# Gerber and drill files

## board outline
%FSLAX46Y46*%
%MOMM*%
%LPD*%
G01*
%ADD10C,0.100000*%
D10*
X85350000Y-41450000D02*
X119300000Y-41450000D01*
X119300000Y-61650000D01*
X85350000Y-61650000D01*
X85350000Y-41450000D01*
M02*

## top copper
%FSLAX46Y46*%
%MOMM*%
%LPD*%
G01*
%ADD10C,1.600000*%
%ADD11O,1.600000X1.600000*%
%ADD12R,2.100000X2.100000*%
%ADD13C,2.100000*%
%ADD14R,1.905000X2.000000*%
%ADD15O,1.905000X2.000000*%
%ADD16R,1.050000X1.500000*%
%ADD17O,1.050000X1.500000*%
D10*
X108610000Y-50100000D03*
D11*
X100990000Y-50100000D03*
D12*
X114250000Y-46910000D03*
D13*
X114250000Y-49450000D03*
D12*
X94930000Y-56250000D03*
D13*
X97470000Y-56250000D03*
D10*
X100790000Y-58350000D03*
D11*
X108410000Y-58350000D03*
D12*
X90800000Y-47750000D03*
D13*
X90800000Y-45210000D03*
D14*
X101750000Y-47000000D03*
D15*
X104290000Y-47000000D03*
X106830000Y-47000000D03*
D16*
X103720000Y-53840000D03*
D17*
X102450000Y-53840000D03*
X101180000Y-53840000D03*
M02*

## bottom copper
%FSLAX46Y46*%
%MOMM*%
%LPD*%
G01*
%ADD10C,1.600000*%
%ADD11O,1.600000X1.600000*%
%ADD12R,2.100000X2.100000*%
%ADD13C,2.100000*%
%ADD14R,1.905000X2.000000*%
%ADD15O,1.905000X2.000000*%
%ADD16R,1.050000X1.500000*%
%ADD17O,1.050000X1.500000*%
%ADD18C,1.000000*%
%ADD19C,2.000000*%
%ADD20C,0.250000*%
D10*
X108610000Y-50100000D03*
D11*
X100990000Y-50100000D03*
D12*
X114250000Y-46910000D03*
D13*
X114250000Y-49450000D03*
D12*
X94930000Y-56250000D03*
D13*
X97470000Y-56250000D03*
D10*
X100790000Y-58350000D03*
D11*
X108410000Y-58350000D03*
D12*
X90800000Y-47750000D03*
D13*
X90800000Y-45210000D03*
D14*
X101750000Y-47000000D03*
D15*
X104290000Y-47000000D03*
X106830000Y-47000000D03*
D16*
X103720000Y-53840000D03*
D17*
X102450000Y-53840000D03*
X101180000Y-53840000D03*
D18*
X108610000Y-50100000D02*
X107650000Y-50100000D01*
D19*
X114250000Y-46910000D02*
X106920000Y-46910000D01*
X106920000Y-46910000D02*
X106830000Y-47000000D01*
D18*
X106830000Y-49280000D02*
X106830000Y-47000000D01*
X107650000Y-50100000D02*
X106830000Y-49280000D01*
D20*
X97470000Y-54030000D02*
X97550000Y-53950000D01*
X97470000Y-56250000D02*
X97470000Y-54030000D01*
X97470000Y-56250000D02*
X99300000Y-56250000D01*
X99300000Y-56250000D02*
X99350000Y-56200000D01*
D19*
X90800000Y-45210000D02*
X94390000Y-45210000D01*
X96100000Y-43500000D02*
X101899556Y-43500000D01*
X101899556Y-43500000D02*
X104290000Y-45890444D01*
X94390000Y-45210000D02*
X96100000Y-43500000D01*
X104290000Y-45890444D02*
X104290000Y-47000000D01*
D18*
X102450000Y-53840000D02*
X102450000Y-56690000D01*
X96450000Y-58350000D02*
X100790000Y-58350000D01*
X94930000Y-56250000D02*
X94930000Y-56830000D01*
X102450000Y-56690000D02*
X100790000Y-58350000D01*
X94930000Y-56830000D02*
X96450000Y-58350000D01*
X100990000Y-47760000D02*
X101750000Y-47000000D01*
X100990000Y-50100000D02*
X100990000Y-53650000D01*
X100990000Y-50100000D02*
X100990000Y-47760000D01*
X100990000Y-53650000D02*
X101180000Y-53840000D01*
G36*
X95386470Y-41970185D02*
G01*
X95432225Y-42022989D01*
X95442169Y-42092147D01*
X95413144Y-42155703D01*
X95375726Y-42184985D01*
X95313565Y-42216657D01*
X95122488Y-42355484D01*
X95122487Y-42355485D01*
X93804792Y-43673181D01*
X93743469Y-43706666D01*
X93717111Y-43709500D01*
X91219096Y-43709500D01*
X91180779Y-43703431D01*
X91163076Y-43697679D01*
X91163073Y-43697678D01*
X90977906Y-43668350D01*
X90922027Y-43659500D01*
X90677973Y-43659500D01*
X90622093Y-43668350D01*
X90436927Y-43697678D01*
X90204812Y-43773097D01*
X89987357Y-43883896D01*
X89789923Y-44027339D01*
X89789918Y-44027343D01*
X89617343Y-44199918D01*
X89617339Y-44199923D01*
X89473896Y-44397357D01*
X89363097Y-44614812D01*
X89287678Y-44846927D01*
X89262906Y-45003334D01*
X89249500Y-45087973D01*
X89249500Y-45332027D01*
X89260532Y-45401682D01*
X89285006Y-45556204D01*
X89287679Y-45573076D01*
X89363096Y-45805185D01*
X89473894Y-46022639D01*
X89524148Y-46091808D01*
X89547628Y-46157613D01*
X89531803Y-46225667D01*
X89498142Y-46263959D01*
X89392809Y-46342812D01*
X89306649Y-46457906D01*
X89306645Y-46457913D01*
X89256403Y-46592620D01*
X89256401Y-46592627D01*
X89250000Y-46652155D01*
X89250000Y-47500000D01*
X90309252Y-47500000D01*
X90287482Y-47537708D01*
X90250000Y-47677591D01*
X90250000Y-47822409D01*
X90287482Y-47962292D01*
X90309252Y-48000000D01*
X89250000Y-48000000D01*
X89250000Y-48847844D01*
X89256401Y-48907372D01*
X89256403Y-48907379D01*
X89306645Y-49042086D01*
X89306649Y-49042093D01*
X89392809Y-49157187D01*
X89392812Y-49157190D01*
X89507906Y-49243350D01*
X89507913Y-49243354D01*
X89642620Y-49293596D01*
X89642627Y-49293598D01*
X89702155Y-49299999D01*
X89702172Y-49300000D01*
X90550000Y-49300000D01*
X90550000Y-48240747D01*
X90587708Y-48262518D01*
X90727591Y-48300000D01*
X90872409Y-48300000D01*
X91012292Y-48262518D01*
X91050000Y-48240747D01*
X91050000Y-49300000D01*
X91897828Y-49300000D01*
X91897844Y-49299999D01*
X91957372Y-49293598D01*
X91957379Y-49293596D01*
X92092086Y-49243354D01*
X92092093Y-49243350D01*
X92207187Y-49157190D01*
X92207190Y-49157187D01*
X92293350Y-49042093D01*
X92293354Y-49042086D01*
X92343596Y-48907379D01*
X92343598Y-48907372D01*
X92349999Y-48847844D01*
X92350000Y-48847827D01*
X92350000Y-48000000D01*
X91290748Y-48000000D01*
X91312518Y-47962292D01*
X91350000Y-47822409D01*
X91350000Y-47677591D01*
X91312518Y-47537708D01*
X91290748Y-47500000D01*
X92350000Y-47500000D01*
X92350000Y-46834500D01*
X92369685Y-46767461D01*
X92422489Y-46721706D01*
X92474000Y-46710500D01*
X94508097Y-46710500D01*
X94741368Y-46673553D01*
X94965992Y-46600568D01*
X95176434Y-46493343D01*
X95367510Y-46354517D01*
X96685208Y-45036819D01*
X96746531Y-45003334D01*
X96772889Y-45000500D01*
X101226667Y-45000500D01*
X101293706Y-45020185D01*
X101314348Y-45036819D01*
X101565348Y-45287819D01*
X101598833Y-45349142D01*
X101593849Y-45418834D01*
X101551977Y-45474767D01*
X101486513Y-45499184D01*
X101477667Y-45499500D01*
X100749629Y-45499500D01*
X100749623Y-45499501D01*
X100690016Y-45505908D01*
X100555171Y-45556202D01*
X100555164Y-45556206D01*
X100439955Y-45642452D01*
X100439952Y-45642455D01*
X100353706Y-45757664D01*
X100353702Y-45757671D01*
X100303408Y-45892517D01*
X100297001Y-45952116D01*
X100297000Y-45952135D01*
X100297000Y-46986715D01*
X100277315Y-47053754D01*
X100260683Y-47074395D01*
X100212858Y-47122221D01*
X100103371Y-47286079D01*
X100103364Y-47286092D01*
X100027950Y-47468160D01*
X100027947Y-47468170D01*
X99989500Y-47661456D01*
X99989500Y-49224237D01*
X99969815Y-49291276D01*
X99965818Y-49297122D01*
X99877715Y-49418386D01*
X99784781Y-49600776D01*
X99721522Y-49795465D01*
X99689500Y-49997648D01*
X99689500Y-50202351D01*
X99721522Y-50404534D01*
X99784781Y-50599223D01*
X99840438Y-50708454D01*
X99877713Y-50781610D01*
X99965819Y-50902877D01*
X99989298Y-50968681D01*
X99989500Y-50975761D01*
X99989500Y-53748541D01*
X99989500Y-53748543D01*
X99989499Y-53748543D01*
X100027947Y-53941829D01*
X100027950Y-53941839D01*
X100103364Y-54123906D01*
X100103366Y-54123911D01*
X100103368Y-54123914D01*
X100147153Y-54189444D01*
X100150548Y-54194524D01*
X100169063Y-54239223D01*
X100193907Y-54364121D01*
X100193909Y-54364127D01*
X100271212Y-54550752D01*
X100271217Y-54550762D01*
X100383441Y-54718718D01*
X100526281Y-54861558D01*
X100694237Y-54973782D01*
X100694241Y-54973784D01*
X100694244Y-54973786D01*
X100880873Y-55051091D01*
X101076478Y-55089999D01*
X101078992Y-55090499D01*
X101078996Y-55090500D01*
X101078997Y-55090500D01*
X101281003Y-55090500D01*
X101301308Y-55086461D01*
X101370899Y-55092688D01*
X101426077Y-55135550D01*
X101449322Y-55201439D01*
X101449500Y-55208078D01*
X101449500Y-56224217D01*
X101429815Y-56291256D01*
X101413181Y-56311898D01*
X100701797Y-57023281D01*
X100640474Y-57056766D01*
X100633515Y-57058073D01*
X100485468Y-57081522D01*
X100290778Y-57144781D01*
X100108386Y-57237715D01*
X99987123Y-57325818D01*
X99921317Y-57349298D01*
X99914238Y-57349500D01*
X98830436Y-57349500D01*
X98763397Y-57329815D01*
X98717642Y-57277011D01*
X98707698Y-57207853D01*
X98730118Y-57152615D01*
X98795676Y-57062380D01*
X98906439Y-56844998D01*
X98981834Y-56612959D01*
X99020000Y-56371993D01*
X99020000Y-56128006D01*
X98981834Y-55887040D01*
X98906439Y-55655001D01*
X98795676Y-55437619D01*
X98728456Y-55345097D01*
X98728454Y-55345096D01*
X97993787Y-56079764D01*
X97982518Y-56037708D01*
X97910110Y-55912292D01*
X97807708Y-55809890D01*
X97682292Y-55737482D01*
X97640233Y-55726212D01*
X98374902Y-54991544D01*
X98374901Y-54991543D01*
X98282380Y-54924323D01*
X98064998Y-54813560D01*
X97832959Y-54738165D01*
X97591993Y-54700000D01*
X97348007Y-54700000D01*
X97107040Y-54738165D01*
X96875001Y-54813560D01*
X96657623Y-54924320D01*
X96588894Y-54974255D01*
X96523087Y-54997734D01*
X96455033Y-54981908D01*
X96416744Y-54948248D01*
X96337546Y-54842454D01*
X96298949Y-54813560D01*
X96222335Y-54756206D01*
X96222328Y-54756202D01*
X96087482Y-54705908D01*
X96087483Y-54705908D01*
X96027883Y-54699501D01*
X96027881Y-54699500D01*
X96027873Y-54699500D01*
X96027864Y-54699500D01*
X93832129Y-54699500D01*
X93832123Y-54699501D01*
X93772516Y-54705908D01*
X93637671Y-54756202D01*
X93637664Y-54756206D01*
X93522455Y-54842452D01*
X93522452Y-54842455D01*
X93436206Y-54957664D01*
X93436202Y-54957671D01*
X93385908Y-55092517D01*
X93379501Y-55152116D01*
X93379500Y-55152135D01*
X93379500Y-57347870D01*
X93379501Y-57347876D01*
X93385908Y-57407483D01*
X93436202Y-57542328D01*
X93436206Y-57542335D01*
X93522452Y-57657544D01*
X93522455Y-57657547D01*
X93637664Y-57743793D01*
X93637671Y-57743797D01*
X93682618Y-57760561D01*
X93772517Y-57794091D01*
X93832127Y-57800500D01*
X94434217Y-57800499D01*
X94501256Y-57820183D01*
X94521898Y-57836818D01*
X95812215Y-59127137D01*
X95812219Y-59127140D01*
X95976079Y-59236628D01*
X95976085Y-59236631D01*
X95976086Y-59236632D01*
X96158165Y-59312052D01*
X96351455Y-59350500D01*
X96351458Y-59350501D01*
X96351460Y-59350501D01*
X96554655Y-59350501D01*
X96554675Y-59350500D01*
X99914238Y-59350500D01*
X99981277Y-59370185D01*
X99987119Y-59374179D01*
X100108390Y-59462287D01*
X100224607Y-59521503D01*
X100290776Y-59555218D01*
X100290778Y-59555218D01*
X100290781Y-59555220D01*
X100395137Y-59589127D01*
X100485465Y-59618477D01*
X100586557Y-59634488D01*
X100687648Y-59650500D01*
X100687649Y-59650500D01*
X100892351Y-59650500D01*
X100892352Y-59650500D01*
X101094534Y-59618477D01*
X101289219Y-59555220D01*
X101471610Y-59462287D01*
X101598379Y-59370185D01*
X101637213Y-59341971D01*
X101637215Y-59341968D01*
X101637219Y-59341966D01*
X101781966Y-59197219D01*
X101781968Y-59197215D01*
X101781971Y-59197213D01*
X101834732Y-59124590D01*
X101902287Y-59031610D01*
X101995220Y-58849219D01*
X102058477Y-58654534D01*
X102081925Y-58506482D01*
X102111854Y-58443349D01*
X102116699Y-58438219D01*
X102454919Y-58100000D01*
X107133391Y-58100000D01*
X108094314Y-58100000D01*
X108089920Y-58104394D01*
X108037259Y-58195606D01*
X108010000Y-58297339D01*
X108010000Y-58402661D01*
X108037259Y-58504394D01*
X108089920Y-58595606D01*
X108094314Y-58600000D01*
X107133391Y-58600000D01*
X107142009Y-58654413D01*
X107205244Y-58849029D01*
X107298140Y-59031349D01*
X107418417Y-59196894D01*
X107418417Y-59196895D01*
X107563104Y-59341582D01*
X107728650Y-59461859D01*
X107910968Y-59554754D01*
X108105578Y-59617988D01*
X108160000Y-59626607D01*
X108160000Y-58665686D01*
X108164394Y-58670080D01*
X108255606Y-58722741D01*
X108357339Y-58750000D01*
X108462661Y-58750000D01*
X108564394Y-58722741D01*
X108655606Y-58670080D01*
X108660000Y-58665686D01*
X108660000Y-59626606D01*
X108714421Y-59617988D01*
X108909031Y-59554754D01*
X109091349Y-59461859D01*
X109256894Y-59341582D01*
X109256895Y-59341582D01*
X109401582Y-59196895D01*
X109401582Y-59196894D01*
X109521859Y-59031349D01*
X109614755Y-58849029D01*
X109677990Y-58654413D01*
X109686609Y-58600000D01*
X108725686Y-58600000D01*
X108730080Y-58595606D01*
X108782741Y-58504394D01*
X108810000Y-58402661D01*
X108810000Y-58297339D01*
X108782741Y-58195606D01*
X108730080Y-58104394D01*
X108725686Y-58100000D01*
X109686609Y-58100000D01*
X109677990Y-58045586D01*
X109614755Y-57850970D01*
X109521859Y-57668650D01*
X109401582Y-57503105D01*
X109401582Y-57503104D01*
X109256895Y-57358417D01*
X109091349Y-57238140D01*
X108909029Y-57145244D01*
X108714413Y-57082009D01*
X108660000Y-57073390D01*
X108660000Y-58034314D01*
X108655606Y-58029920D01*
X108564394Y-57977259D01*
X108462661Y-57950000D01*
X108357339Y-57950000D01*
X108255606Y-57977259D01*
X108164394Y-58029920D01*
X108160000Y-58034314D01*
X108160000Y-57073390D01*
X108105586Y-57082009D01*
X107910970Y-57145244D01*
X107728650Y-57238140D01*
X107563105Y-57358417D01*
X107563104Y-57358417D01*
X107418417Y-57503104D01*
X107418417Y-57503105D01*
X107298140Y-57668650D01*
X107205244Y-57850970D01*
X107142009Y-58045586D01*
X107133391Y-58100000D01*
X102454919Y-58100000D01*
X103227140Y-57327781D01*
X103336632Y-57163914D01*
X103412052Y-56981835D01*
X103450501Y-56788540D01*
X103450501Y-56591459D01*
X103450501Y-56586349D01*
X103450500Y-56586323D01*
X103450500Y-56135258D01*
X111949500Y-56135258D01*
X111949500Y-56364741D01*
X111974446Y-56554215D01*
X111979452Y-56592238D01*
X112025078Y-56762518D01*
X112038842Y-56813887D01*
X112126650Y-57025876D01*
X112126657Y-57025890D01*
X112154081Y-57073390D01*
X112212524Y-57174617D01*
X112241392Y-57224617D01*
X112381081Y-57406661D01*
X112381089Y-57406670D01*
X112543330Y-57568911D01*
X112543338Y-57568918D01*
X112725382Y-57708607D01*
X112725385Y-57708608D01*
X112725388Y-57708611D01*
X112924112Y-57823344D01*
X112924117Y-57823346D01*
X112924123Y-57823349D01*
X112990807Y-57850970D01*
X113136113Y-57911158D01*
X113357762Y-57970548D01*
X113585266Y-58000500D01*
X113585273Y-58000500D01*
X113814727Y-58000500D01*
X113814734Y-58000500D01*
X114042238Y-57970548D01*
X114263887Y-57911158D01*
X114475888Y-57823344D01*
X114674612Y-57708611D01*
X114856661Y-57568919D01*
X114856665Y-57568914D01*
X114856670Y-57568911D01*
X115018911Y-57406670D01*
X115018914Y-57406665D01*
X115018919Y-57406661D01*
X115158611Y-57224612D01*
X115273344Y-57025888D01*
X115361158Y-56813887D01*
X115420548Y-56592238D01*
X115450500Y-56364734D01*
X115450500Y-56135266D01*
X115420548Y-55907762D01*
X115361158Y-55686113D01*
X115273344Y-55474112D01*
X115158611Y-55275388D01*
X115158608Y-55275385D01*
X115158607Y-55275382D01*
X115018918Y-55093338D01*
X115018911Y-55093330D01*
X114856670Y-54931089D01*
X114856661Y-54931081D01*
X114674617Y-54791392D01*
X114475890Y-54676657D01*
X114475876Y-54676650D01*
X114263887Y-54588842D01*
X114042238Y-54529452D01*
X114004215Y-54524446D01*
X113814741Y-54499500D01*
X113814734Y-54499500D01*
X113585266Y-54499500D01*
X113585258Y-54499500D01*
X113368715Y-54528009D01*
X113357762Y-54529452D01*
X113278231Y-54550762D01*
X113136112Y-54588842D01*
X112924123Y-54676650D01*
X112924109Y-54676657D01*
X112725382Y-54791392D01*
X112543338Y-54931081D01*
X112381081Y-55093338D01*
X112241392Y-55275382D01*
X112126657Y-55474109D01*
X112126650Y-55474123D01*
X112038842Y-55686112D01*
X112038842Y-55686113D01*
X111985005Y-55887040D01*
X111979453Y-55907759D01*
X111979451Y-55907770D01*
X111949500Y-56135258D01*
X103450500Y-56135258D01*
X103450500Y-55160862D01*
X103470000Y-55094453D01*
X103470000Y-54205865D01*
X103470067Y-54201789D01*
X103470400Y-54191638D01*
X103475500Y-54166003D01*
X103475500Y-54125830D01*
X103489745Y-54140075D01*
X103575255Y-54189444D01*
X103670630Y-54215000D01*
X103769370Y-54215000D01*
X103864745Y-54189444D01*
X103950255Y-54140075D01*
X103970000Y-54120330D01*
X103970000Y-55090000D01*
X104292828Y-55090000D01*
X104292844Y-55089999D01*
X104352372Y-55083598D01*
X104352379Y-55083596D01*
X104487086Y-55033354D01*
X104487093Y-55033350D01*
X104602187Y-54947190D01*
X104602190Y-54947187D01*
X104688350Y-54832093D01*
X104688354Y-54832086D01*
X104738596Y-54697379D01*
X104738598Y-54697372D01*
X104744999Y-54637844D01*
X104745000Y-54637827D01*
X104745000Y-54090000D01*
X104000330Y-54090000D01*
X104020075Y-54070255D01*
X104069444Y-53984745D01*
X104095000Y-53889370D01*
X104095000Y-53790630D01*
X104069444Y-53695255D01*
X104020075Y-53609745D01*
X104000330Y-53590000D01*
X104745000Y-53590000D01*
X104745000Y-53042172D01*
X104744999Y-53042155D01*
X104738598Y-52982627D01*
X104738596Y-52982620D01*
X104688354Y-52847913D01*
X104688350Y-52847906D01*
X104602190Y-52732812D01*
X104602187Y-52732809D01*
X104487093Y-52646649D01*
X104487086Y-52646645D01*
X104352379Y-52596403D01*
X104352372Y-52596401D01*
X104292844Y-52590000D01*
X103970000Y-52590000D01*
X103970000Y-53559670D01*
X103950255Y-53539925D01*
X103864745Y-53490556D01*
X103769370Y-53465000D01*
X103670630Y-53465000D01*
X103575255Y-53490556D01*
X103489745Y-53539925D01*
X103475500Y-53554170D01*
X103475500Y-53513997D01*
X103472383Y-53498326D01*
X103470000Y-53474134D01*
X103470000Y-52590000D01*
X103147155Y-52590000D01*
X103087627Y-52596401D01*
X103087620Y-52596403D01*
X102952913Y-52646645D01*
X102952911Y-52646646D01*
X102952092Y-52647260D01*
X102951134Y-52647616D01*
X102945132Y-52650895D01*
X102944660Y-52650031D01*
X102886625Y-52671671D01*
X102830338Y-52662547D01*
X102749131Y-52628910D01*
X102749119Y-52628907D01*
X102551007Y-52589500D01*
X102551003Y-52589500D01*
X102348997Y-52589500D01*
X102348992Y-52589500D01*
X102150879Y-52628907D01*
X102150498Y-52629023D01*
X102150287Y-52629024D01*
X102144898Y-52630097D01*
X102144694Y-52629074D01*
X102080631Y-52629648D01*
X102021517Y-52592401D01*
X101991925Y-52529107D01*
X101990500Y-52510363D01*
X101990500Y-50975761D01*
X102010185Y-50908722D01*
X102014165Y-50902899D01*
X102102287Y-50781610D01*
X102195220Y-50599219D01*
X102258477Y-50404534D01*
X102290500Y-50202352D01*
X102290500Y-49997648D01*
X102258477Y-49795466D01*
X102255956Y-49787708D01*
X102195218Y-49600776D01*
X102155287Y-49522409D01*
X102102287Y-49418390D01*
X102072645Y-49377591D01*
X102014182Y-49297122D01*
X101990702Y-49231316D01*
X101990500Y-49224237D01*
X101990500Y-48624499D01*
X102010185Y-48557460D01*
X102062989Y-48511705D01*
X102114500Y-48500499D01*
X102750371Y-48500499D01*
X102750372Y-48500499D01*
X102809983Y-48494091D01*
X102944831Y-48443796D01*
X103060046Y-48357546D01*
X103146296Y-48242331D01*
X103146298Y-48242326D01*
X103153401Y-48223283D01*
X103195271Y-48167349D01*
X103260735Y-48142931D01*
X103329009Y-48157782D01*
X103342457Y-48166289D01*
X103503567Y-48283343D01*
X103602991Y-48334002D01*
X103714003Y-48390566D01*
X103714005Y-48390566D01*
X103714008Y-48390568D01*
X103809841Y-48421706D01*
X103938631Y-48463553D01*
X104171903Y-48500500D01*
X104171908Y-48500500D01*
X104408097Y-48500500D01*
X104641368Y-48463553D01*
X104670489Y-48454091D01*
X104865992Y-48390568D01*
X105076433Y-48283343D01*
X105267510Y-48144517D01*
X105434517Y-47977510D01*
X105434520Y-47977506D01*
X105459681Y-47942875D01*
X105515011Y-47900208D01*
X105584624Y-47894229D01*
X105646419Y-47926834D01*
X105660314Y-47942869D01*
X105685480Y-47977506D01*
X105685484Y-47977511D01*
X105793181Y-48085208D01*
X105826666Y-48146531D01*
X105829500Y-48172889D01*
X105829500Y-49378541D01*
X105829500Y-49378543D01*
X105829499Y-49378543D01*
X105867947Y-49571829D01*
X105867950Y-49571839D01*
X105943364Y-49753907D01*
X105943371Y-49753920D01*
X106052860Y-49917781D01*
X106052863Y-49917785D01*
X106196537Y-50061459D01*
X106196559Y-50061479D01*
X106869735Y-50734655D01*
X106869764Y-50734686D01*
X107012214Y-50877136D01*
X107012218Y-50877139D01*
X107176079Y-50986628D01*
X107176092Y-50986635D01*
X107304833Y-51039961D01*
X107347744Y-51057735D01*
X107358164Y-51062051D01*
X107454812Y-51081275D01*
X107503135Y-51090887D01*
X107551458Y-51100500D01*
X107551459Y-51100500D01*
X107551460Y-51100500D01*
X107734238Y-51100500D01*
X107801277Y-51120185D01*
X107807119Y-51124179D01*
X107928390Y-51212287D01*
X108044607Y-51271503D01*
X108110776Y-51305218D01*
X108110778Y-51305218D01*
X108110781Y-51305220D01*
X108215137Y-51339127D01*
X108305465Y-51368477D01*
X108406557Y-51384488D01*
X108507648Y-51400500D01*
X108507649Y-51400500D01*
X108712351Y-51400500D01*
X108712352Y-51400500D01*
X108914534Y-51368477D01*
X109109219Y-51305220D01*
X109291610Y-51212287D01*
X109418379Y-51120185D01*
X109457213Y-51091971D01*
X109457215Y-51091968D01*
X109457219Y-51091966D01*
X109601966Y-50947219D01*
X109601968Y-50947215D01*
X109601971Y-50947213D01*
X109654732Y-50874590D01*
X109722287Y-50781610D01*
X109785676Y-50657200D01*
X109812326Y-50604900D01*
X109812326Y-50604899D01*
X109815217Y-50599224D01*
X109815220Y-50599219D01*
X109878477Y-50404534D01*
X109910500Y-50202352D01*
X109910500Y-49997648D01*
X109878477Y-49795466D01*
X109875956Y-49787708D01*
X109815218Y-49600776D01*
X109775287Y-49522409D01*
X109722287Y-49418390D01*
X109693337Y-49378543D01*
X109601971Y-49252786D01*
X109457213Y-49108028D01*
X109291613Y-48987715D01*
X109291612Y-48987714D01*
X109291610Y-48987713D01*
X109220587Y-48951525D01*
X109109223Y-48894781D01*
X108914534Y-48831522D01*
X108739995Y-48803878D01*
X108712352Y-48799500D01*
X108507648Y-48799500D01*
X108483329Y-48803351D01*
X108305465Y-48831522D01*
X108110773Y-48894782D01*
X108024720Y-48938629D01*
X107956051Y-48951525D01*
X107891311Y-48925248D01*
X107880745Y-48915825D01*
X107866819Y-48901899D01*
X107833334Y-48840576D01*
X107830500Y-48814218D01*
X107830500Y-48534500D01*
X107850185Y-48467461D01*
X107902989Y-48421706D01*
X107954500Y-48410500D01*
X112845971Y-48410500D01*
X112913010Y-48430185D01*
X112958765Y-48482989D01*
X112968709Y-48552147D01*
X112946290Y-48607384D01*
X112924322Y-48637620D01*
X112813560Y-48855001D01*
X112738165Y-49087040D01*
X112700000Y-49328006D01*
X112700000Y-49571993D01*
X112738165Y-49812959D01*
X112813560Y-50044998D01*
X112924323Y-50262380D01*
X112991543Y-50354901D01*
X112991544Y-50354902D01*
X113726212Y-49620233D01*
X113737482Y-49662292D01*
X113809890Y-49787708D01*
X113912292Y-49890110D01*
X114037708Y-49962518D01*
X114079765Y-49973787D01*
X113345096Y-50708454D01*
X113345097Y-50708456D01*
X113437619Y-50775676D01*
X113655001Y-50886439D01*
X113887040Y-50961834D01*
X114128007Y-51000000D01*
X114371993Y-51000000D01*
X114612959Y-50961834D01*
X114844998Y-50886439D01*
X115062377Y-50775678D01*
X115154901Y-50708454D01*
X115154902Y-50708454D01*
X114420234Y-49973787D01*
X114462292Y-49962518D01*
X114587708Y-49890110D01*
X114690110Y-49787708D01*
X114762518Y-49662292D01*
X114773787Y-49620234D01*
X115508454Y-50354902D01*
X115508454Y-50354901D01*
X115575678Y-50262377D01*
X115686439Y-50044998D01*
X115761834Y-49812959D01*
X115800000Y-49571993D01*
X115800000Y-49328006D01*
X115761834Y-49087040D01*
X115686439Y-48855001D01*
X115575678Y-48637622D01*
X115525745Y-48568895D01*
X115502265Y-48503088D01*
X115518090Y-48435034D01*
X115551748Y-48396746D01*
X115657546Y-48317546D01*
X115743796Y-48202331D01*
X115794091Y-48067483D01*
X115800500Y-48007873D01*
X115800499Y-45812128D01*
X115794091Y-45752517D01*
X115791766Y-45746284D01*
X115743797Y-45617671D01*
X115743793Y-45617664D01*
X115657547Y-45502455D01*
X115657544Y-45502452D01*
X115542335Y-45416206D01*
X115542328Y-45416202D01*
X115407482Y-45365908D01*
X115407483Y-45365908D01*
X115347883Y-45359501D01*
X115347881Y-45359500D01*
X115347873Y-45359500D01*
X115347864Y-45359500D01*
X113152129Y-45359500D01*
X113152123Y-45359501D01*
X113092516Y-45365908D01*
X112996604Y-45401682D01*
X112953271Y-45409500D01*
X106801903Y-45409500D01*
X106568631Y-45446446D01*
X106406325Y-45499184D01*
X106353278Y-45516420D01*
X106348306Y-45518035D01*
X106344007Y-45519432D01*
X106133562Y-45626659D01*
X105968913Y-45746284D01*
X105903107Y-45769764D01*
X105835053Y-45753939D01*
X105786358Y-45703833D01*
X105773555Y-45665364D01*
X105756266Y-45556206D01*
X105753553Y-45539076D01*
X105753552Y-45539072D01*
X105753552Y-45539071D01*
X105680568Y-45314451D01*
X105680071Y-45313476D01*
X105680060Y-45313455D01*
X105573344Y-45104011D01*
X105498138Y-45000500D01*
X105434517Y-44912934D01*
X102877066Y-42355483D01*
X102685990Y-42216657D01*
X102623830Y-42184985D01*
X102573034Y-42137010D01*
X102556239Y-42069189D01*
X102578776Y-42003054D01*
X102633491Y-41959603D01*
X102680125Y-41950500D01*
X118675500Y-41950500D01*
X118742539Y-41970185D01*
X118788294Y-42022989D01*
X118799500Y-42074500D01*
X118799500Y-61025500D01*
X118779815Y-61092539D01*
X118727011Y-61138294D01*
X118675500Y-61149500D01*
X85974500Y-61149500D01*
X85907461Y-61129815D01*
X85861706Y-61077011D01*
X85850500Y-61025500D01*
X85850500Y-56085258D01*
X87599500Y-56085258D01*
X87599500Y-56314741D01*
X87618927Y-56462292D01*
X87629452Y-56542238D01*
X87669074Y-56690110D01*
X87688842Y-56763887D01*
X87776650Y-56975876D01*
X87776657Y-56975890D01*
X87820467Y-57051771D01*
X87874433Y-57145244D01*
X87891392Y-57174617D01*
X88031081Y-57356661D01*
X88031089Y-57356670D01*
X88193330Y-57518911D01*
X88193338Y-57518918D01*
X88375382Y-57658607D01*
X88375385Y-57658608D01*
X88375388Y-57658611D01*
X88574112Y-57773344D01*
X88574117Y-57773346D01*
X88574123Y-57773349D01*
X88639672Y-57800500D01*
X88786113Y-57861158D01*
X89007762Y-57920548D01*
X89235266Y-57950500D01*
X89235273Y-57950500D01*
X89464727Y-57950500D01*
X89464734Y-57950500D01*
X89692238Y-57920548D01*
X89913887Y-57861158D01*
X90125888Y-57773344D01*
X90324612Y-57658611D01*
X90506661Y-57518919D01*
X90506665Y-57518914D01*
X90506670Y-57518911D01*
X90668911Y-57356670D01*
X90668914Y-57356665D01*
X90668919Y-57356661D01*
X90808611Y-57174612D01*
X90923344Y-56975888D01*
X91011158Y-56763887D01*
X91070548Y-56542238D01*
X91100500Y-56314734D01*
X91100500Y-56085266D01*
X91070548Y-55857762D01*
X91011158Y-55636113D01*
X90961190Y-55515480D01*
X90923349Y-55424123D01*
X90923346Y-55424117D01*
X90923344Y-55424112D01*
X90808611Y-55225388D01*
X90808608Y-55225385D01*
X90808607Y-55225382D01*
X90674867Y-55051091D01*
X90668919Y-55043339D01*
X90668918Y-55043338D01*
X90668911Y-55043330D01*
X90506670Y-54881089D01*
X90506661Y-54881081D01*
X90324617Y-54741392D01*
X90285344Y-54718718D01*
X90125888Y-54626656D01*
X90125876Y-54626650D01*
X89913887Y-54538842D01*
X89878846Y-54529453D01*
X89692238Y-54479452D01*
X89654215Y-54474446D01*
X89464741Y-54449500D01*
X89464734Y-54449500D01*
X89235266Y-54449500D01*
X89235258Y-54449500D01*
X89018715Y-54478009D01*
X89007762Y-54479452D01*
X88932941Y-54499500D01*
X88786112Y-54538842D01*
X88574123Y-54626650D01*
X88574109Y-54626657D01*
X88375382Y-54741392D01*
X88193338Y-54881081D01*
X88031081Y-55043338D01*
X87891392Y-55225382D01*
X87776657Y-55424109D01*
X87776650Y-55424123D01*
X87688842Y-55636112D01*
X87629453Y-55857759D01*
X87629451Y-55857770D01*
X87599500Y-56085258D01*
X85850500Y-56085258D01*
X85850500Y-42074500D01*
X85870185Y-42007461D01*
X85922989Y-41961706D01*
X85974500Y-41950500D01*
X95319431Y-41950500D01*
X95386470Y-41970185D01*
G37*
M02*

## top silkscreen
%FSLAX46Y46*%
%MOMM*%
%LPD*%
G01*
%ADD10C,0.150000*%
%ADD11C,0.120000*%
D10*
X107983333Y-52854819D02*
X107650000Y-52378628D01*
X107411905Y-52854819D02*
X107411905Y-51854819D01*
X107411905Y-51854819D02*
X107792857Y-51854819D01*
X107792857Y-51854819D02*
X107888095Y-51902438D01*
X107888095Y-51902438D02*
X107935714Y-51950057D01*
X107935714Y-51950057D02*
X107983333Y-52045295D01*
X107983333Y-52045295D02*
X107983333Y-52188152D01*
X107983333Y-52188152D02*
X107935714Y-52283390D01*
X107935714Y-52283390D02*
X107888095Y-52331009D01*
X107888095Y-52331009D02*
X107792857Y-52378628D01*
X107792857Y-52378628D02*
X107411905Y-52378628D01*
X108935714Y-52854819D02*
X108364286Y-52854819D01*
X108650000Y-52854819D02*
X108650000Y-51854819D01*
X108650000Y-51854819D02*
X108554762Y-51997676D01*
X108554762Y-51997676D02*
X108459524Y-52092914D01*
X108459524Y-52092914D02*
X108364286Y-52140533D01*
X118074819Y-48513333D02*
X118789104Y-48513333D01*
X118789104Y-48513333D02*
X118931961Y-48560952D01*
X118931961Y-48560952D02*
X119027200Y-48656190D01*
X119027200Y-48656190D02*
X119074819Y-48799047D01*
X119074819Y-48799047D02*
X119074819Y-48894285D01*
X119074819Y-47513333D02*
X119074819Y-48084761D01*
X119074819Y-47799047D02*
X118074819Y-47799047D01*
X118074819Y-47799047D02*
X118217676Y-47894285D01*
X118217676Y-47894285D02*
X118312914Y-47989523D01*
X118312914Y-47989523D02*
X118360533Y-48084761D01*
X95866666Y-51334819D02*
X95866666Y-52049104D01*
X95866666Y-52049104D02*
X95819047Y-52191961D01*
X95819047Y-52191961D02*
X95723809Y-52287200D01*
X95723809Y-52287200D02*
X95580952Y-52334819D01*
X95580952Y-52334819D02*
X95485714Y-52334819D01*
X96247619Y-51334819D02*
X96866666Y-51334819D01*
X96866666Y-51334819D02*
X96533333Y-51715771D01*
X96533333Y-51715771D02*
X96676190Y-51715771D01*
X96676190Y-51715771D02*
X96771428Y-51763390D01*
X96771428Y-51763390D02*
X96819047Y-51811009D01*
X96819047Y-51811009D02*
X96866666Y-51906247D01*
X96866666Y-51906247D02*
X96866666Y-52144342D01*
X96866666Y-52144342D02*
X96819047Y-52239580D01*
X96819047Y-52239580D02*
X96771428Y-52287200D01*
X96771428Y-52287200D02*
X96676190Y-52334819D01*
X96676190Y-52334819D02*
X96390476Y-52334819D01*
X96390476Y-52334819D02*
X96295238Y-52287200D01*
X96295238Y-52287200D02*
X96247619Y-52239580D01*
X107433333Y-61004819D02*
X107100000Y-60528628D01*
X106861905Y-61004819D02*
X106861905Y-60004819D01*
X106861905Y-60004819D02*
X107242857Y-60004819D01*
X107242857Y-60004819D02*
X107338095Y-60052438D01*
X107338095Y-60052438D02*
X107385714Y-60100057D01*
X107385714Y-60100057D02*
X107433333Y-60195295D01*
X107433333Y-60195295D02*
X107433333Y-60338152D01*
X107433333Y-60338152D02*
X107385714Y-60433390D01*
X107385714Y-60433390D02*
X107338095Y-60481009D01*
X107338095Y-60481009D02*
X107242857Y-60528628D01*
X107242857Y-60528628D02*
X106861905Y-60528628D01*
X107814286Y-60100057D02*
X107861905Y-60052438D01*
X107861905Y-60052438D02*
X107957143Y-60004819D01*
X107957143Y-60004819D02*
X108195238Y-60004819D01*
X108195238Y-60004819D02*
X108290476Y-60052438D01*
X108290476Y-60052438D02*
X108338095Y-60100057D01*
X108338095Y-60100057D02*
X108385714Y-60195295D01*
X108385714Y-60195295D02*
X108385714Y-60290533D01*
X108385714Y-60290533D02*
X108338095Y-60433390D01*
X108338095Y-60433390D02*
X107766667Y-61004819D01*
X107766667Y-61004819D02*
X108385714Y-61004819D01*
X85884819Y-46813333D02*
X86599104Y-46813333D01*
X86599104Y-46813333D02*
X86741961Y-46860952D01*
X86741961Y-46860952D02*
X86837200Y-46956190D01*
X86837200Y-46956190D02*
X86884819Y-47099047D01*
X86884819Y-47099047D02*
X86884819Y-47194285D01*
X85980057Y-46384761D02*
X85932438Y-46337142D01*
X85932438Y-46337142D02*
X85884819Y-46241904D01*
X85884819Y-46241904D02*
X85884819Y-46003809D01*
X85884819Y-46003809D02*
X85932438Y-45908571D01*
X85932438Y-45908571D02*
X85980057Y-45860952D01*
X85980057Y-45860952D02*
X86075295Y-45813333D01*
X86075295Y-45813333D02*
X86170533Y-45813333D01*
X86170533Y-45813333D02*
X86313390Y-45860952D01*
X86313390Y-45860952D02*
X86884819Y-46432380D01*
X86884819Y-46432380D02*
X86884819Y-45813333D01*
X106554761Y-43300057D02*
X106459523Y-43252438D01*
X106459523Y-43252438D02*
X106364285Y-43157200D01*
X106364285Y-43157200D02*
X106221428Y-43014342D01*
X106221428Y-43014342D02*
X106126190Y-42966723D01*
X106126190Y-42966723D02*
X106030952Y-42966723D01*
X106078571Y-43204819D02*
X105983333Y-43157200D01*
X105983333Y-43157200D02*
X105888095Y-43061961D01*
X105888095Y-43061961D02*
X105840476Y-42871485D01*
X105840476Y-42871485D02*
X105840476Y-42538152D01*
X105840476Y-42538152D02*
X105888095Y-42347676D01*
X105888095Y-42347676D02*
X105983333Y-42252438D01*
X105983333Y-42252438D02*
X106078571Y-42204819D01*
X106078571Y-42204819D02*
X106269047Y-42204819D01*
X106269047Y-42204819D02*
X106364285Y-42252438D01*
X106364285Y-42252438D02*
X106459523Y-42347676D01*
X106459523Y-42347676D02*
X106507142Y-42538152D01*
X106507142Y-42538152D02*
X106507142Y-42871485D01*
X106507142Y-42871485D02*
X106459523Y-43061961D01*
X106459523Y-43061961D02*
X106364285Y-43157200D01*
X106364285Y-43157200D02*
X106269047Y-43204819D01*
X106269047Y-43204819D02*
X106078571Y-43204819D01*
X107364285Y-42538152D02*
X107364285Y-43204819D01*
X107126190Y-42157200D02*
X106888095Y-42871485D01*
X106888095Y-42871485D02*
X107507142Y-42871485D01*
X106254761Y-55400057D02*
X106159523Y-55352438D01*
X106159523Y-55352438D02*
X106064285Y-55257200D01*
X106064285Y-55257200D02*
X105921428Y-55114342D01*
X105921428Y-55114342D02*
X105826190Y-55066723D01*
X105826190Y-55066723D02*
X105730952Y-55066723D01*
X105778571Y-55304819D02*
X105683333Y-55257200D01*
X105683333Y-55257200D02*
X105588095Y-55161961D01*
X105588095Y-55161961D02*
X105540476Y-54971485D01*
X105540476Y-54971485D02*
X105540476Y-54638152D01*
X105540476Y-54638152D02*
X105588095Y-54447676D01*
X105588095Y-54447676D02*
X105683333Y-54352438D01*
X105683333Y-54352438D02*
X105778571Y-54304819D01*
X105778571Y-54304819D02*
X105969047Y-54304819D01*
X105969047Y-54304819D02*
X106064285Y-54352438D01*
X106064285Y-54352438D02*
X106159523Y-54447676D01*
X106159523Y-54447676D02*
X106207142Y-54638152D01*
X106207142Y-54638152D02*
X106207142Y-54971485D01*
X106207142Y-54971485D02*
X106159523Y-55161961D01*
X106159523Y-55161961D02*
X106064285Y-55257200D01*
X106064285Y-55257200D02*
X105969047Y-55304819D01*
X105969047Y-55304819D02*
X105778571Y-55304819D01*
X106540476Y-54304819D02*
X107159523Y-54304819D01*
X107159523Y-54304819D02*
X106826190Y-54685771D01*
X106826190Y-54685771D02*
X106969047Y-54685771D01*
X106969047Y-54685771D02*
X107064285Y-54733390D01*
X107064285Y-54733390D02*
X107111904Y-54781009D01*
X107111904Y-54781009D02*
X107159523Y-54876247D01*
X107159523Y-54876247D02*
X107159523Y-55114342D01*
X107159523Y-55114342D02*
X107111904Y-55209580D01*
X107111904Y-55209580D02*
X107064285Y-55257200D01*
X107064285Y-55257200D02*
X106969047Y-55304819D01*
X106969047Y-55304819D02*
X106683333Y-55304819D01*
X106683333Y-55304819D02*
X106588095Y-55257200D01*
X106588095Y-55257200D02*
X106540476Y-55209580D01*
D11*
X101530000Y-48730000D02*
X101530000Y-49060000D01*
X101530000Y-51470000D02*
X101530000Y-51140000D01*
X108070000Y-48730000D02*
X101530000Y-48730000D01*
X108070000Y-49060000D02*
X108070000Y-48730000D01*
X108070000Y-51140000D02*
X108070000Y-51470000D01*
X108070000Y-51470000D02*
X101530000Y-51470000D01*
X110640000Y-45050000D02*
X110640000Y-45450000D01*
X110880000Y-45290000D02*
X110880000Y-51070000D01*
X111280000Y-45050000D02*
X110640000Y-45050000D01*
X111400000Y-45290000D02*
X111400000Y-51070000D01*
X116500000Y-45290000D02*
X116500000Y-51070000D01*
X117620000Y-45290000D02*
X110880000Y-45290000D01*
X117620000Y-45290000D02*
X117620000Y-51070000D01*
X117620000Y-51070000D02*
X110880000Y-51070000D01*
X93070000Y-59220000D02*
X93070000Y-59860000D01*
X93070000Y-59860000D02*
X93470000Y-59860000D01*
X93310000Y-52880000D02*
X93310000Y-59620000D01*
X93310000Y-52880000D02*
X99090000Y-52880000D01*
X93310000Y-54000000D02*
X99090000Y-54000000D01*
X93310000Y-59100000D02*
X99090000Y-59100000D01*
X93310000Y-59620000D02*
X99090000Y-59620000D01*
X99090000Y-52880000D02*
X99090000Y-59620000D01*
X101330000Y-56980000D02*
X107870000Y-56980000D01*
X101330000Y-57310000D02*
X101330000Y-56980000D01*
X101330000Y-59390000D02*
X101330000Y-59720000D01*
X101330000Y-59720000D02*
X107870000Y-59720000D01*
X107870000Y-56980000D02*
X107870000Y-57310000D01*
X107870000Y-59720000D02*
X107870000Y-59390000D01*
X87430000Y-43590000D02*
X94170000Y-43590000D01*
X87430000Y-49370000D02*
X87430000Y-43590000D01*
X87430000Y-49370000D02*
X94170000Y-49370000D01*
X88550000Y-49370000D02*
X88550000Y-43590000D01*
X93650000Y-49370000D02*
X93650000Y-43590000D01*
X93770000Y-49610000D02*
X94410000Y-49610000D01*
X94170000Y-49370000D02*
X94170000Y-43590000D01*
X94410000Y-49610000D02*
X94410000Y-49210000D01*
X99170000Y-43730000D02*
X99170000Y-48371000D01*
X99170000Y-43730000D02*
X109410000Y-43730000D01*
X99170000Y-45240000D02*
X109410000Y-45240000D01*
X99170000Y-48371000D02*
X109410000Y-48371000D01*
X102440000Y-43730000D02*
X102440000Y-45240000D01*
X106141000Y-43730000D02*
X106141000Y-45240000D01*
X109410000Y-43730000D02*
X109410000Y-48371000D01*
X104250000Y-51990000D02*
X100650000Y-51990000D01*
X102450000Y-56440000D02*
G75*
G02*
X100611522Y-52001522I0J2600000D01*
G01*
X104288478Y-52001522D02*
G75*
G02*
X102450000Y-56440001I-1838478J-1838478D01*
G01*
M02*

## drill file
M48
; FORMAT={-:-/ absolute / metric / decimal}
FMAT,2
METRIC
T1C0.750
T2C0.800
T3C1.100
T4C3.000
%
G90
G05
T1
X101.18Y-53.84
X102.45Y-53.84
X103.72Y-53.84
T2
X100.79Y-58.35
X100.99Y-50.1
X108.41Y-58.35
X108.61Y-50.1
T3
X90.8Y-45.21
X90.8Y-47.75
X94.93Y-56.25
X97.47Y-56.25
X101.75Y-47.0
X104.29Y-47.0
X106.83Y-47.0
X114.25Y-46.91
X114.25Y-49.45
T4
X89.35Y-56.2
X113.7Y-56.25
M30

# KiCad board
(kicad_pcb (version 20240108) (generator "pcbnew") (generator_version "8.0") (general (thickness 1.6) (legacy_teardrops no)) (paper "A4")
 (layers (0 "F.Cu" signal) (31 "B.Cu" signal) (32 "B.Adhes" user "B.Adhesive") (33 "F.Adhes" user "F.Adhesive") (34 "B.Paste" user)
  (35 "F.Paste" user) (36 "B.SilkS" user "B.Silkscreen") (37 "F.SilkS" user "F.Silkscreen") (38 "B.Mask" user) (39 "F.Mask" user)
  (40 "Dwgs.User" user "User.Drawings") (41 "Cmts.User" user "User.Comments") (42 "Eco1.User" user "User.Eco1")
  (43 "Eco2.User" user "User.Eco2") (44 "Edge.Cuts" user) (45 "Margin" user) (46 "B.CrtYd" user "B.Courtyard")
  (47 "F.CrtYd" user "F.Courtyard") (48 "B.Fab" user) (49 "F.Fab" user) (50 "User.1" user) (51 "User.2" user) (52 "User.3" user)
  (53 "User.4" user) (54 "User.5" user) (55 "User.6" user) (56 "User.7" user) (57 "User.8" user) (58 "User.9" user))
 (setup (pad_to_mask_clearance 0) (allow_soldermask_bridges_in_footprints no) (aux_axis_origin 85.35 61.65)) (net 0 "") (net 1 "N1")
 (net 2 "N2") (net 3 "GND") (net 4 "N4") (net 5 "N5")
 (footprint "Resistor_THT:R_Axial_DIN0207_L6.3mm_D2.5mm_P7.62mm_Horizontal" (layer "F.Cu") (at 108.61 50.1 180)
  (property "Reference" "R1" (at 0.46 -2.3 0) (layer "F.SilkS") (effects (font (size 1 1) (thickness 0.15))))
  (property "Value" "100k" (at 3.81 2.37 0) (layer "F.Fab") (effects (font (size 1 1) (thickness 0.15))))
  (fp_line (start 7.08 1.37) (end 7.08 1.04) (stroke (width 0.12) (type solid)) (layer "F.SilkS"))
  (fp_line (start 7.08 -1.37) (end 7.08 -1.04) (stroke (width 0.12) (type solid)) (layer "F.SilkS"))
  (fp_line (start 0.54 1.37) (end 7.08 1.37) (stroke (width 0.12) (type solid)) (layer "F.SilkS"))
  (fp_line (start 0.54 1.04) (end 0.54 1.37) (stroke (width 0.12) (type solid)) (layer "F.SilkS"))
  (fp_line (start 0.54 -1.04) (end 0.54 -1.37) (stroke (width 0.12) (type solid)) (layer "F.SilkS"))
  (fp_line (start 0.54 -1.37) (end 7.08 -1.37) (stroke (width 0.12) (type solid)) (layer "F.SilkS"))
  (pad "1" thru_hole circle (at 0 0 180) (size 1.6 1.6) (drill 0.8) (layers "*.Cu" "*.Mask") (remove_unused_layers no) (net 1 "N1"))
  (pad "2" thru_hole oval (at 7.62 0 180) (size 1.6 1.6) (drill 0.8) (layers "*.Cu" "*.Mask") (remove_unused_layers no) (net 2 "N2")))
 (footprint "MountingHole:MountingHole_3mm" (layer "F.Cu") (at 113.7 56.25)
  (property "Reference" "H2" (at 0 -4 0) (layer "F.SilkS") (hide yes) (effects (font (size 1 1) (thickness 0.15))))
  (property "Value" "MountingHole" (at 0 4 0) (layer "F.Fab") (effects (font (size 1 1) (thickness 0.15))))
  (pad "" np_thru_hole circle (at 0 0) (size 3 3) (drill 3) (layers "*.Cu" "*.Mask")))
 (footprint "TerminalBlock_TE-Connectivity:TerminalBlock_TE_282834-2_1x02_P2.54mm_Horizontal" (layer "F.Cu") (at 114.25 46.91 -90)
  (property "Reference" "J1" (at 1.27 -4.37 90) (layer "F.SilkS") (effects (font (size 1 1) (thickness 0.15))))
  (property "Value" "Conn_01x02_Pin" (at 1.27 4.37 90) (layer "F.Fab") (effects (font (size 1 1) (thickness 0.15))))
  (fp_line (start -1.86 3.61) (end -1.46 3.61) (stroke (width 0.12) (type solid)) (layer "F.SilkS"))
  (fp_line (start -1.62 3.37) (end 4.16 3.37) (stroke (width 0.12) (type solid)) (layer "F.SilkS"))
  (fp_line (start -1.86 2.97) (end -1.86 3.61) (stroke (width 0.12) (type solid)) (layer "F.SilkS"))
  (fp_line (start -1.62 2.85) (end 4.16 2.85) (stroke (width 0.12) (type solid)) (layer "F.SilkS"))
  (fp_line (start -1.62 -2.25) (end 4.16 -2.25) (stroke (width 0.12) (type solid)) (layer "F.SilkS"))
  (fp_line (start -1.62 -3.37) (end -1.62 3.37) (stroke (width 0.12) (type solid)) (layer "F.SilkS"))
  (fp_line (start -1.62 -3.37) (end 4.16 -3.37) (stroke (width 0.12) (type solid)) (layer "F.SilkS"))
  (fp_line (start 4.16 -3.37) (end 4.16 3.37) (stroke (width 0.12) (type solid)) (layer "F.SilkS"))
  (pad "1" thru_hole rect (at 0 0 270) (size 2.1 2.1) (drill 1.1) (layers "*.Cu" "*.Mask") (remove_unused_layers no) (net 1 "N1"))
  (pad "2" thru_hole circle (at 2.54 0 270) (size 2.1 2.1) (drill 1.1) (layers "*.Cu" "*.Mask") (remove_unused_layers no) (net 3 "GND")))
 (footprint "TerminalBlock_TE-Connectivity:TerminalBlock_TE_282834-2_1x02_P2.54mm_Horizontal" (layer "F.Cu") (at 94.93 56.25)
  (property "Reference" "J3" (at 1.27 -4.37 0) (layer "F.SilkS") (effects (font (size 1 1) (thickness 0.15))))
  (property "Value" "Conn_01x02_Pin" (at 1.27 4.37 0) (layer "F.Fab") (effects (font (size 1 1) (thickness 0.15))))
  (fp_line (start -1.86 2.97) (end -1.86 3.61) (stroke (width 0.12) (type solid)) (layer "F.SilkS"))
  (fp_line (start -1.86 3.61) (end -1.46 3.61) (stroke (width 0.12) (type solid)) (layer "F.SilkS"))
  (fp_line (start -1.62 -3.37) (end -1.62 3.37) (stroke (width 0.12) (type solid)) (layer "F.SilkS"))
  (fp_line (start -1.62 -3.37) (end 4.16 -3.37) (stroke (width 0.12) (type solid)) (layer "F.SilkS"))
  (fp_line (start -1.62 -2.25) (end 4.16 -2.25) (stroke (width 0.12) (type solid)) (layer "F.SilkS"))
  (fp_line (start -1.62 2.85) (end 4.16 2.85) (stroke (width 0.12) (type solid)) (layer "F.SilkS"))
  (fp_line (start -1.62 3.37) (end 4.16 3.37) (stroke (width 0.12) (type solid)) (layer "F.SilkS"))
  (fp_line (start 4.16 -3.37) (end 4.16 3.37) (stroke (width 0.12) (type solid)) (layer "F.SilkS"))
  (pad "1" thru_hole rect (at 0 0) (size 2.1 2.1) (drill 1.1) (layers "*.Cu" "*.Mask") (remove_unused_layers no) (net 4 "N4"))
  (pad "2" thru_hole circle (at 2.54 0) (size 2.1 2.1) (drill 1.1) (layers "*.Cu" "*.Mask") (remove_unused_layers no) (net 3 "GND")))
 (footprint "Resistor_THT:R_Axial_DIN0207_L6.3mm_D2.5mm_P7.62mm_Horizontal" (layer "F.Cu") (at 100.79 58.35)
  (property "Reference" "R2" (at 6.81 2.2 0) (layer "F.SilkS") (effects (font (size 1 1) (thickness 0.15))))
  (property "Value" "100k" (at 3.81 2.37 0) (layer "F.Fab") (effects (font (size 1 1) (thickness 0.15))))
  (fp_line (start 0.54 -1.37) (end 7.08 -1.37) (stroke (width 0.12) (type solid)) (layer "F.SilkS"))
  (fp_line (start 0.54 -1.04) (end 0.54 -1.37) (stroke (width 0.12) (type solid)) (layer "F.SilkS"))
  (fp_line (start 0.54 1.04) (end 0.54 1.37) (stroke (width 0.12) (type solid)) (layer "F.SilkS"))
  (fp_line (start 0.54 1.37) (end 7.08 1.37) (stroke (width 0.12) (type solid)) (layer "F.SilkS"))
  (fp_line (start 7.08 -1.37) (end 7.08 -1.04) (stroke (width 0.12) (type solid)) (layer "F.SilkS"))
  (fp_line (start 7.08 1.37) (end 7.08 1.04) (stroke (width 0.12) (type solid)) (layer "F.SilkS"))
  (pad "1" thru_hole circle (at 0 0) (size 1.6 1.6) (drill 0.8) (layers "*.Cu" "*.Mask") (remove_unused_layers no) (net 4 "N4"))
  (pad "2" thru_hole oval (at 7.62 0) (size 1.6 1.6) (drill 0.8) (layers "*.Cu" "*.Mask") (remove_unused_layers no) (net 3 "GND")))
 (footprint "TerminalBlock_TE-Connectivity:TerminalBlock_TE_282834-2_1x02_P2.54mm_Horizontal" (layer "F.Cu") (at 90.8 47.75 90)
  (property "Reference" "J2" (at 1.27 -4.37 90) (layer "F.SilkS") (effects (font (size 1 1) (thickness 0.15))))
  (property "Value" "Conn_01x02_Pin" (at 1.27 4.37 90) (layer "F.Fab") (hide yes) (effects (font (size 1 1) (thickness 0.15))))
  (fp_line (start 4.16 -3.37) (end 4.16 3.37) (stroke (width 0.12) (type solid)) (layer "F.SilkS"))
  (fp_line (start -1.62 -3.37) (end 4.16 -3.37) (stroke (width 0.12) (type solid)) (layer "F.SilkS"))
  (fp_line (start -1.62 -3.37) (end -1.62 3.37) (stroke (width 0.12) (type solid)) (layer "F.SilkS"))
  (fp_line (start -1.62 -2.25) (end 4.16 -2.25) (stroke (width 0.12) (type solid)) (layer "F.SilkS"))
  (fp_line (start -1.62 2.85) (end 4.16 2.85) (stroke (width 0.12) (type solid)) (layer "F.SilkS"))
  (fp_line (start -1.86 2.97) (end -1.86 3.61) (stroke (width 0.12) (type solid)) (layer "F.SilkS"))
  (fp_line (start -1.62 3.37) (end 4.16 3.37) (stroke (width 0.12) (type solid)) (layer "F.SilkS"))
  (fp_line (start -1.86 3.61) (end -1.46 3.61) (stroke (width 0.12) (type solid)) (layer "F.SilkS"))
  (pad "1" thru_hole rect (at 0 0 90) (size 2.1 2.1) (drill 1.1) (layers "*.Cu" "*.Mask") (remove_unused_layers no) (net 3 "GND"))
  (pad "2" thru_hole circle (at 2.54 0 90) (size 2.1 2.1) (drill 1.1) (layers "*.Cu" "*.Mask") (remove_unused_layers no) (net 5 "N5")))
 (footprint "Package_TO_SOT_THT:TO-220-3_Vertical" (layer "F.Cu") (at 101.75 47)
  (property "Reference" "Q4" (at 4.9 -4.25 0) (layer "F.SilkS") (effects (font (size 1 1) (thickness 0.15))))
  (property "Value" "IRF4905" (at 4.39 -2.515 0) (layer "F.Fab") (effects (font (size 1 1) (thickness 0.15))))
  (fp_line (start -2.58 -3.27) (end -2.58 1.371) (stroke (width 0.12) (type solid)) (layer "F.SilkS"))
  (fp_line (start -2.58 -3.27) (end 7.66 -3.27) (stroke (width 0.12) (type solid)) (layer "F.SilkS"))
  (fp_line (start -2.58 -1.76) (end 7.66 -1.76) (stroke (width 0.12) (type solid)) (layer "F.SilkS"))
  (fp_line (start -2.58 1.371) (end 7.66 1.371) (stroke (width 0.12) (type solid)) (layer "F.SilkS"))
  (fp_line (start 0.69 -3.27) (end 0.69 -1.76) (stroke (width 0.12) (type solid)) (layer "F.SilkS"))
  (fp_line (start 4.391 -3.27) (end 4.391 -1.76) (stroke (width 0.12) (type solid)) (layer "F.SilkS"))
  (fp_line (start 7.66 -3.27) (end 7.66 1.371) (stroke (width 0.12) (type solid)) (layer "F.SilkS"))
  (pad "1" thru_hole rect (at 0 0) (size 1.905 2) (drill 1.1) (layers "*.Cu" "*.Mask") (remove_unused_layers no) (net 2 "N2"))
  (pad "2" thru_hole oval (at 2.54 0) (size 1.905 2) (drill 1.1) (layers "*.Cu" "*.Mask") (remove_unused_layers no) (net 5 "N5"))
  (pad "3" thru_hole oval (at 5.08 0) (size 1.905 2) (drill 1.1) (layers "*.Cu" "*.Mask") (remove_unused_layers no) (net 1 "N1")))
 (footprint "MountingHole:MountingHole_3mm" (layer "F.Cu") (at 89.35 56.2)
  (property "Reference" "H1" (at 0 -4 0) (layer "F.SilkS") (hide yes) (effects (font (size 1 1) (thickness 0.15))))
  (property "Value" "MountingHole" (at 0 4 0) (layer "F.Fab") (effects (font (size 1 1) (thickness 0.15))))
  (pad "" np_thru_hole circle (at 0 0) (size 3 3) (drill 3) (layers "*.Cu" "*.Mask")))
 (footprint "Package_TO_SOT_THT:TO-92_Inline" (layer "F.Cu") (at 103.72 53.84 180)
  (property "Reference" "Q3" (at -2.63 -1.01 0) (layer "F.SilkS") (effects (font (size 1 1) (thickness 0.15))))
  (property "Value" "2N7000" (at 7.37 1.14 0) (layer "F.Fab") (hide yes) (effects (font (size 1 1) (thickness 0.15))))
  (fp_line (start -0.53 1.85) (end 3.07 1.85) (stroke (width 0.12) (type solid)) (layer "F.SilkS"))
  (fp_arc (start 1.27 -2.6) (mid 3.672087 -0.994977) (end 3.108478 1.838478) (stroke (width 0.12) (type solid)) (layer "F.SilkS"))
  (fp_arc (start -0.568478 1.838478) (mid -1.132087 -0.994977) (end 1.27 -2.6) (stroke (width 0.12) (type solid)) (layer "F.SilkS"))
  (pad "1" thru_hole rect (at 0 0 180) (size 1.05 1.5) (drill 0.75) (layers "*.Cu" "*.Mask") (remove_unused_layers no) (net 3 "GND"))
  (pad "2" thru_hole oval (at 1.27 0 180) (size 1.05 1.5) (drill 0.75) (layers "*.Cu" "*.Mask") (remove_unused_layers no) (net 4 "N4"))
  (pad "3" thru_hole oval (at 2.54 0 180) (size 1.05 1.5) (drill 0.75) (layers "*.Cu" "*.Mask") (remove_unused_layers no) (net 2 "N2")))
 (gr_rect (start 85.35 41.45) (end 119.3 61.65) (stroke (width 0.1) (type default)) (fill none) (layer "Edge.Cuts"))
 (segment (start 108.61 50.1) (end 107.65 50.1) (width 1) (layer "B.Cu") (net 1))
 (segment (start 114.25 46.91) (end 106.92 46.91) (width 2) (layer "B.Cu") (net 1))
 (segment (start 106.92 46.91) (end 106.83 47) (width 2) (layer "B.Cu") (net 1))
 (segment (start 106.83 49.28) (end 106.83 47) (width 1) (layer "B.Cu") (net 1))
 (segment (start 107.65 50.1) (end 106.83 49.28) (width 1) (layer "B.Cu") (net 1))
 (segment (start 97.47 54.03) (end 97.55 53.95) (width 0.25) (layer "B.Cu") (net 3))
 (segment (start 97.47 56.25) (end 97.47 54.03) (width 0.25) (layer "B.Cu") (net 3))
 (segment (start 97.47 56.25) (end 99.3 56.25) (width 0.25) (layer "B.Cu") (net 3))
 (segment (start 99.3 56.25) (end 99.35 56.2) (width 0.25) (layer "B.Cu") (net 3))
 (segment (start 90.8 45.21) (end 94.39 45.21) (width 2) (layer "B.Cu") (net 5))
 (segment (start 96.1 43.5) (end 101.899556 43.5) (width 2) (layer "B.Cu") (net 5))
 (segment (start 101.899556 43.5) (end 104.29 45.890444) (width 2) (layer "B.Cu") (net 5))
 (segment (start 94.39 45.21) (end 96.1 43.5) (width 2) (layer "B.Cu") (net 5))
 (segment (start 104.29 45.890444) (end 104.29 47) (width 2) (layer "B.Cu") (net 5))
 (segment (start 102.45 53.84) (end 102.45 56.69) (width 1) (layer "B.Cu") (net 4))
 (segment (start 96.45 58.35) (end 100.79 58.35) (width 1) (layer "B.Cu") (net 4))
 (segment (start 94.93 56.25) (end 94.93 56.83) (width 1) (layer "B.Cu") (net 4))
 (segment (start 102.45 56.69) (end 100.79 58.35) (width 1) (layer "B.Cu") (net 4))
 (segment (start 94.93 56.83) (end 96.45 58.35) (width 1) (layer "B.Cu") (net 4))
 (segment (start 100.99 47.76) (end 101.75 47) (width 1) (layer "B.Cu") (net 2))
 (segment (start 100.99 50.1) (end 100.99 53.65) (width 1) (layer "B.Cu") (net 2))
 (segment (start 100.99 50.1) (end 100.99 47.76) (width 1) (layer "B.Cu") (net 2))
 (segment (start 100.99 53.65) (end 101.18 53.84) (width 1) (layer "B.Cu") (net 2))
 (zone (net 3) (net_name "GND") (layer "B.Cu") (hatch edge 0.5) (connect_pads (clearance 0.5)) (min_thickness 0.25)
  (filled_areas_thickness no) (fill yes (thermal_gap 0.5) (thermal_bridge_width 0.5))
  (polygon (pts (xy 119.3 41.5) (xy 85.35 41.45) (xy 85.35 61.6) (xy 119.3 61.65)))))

